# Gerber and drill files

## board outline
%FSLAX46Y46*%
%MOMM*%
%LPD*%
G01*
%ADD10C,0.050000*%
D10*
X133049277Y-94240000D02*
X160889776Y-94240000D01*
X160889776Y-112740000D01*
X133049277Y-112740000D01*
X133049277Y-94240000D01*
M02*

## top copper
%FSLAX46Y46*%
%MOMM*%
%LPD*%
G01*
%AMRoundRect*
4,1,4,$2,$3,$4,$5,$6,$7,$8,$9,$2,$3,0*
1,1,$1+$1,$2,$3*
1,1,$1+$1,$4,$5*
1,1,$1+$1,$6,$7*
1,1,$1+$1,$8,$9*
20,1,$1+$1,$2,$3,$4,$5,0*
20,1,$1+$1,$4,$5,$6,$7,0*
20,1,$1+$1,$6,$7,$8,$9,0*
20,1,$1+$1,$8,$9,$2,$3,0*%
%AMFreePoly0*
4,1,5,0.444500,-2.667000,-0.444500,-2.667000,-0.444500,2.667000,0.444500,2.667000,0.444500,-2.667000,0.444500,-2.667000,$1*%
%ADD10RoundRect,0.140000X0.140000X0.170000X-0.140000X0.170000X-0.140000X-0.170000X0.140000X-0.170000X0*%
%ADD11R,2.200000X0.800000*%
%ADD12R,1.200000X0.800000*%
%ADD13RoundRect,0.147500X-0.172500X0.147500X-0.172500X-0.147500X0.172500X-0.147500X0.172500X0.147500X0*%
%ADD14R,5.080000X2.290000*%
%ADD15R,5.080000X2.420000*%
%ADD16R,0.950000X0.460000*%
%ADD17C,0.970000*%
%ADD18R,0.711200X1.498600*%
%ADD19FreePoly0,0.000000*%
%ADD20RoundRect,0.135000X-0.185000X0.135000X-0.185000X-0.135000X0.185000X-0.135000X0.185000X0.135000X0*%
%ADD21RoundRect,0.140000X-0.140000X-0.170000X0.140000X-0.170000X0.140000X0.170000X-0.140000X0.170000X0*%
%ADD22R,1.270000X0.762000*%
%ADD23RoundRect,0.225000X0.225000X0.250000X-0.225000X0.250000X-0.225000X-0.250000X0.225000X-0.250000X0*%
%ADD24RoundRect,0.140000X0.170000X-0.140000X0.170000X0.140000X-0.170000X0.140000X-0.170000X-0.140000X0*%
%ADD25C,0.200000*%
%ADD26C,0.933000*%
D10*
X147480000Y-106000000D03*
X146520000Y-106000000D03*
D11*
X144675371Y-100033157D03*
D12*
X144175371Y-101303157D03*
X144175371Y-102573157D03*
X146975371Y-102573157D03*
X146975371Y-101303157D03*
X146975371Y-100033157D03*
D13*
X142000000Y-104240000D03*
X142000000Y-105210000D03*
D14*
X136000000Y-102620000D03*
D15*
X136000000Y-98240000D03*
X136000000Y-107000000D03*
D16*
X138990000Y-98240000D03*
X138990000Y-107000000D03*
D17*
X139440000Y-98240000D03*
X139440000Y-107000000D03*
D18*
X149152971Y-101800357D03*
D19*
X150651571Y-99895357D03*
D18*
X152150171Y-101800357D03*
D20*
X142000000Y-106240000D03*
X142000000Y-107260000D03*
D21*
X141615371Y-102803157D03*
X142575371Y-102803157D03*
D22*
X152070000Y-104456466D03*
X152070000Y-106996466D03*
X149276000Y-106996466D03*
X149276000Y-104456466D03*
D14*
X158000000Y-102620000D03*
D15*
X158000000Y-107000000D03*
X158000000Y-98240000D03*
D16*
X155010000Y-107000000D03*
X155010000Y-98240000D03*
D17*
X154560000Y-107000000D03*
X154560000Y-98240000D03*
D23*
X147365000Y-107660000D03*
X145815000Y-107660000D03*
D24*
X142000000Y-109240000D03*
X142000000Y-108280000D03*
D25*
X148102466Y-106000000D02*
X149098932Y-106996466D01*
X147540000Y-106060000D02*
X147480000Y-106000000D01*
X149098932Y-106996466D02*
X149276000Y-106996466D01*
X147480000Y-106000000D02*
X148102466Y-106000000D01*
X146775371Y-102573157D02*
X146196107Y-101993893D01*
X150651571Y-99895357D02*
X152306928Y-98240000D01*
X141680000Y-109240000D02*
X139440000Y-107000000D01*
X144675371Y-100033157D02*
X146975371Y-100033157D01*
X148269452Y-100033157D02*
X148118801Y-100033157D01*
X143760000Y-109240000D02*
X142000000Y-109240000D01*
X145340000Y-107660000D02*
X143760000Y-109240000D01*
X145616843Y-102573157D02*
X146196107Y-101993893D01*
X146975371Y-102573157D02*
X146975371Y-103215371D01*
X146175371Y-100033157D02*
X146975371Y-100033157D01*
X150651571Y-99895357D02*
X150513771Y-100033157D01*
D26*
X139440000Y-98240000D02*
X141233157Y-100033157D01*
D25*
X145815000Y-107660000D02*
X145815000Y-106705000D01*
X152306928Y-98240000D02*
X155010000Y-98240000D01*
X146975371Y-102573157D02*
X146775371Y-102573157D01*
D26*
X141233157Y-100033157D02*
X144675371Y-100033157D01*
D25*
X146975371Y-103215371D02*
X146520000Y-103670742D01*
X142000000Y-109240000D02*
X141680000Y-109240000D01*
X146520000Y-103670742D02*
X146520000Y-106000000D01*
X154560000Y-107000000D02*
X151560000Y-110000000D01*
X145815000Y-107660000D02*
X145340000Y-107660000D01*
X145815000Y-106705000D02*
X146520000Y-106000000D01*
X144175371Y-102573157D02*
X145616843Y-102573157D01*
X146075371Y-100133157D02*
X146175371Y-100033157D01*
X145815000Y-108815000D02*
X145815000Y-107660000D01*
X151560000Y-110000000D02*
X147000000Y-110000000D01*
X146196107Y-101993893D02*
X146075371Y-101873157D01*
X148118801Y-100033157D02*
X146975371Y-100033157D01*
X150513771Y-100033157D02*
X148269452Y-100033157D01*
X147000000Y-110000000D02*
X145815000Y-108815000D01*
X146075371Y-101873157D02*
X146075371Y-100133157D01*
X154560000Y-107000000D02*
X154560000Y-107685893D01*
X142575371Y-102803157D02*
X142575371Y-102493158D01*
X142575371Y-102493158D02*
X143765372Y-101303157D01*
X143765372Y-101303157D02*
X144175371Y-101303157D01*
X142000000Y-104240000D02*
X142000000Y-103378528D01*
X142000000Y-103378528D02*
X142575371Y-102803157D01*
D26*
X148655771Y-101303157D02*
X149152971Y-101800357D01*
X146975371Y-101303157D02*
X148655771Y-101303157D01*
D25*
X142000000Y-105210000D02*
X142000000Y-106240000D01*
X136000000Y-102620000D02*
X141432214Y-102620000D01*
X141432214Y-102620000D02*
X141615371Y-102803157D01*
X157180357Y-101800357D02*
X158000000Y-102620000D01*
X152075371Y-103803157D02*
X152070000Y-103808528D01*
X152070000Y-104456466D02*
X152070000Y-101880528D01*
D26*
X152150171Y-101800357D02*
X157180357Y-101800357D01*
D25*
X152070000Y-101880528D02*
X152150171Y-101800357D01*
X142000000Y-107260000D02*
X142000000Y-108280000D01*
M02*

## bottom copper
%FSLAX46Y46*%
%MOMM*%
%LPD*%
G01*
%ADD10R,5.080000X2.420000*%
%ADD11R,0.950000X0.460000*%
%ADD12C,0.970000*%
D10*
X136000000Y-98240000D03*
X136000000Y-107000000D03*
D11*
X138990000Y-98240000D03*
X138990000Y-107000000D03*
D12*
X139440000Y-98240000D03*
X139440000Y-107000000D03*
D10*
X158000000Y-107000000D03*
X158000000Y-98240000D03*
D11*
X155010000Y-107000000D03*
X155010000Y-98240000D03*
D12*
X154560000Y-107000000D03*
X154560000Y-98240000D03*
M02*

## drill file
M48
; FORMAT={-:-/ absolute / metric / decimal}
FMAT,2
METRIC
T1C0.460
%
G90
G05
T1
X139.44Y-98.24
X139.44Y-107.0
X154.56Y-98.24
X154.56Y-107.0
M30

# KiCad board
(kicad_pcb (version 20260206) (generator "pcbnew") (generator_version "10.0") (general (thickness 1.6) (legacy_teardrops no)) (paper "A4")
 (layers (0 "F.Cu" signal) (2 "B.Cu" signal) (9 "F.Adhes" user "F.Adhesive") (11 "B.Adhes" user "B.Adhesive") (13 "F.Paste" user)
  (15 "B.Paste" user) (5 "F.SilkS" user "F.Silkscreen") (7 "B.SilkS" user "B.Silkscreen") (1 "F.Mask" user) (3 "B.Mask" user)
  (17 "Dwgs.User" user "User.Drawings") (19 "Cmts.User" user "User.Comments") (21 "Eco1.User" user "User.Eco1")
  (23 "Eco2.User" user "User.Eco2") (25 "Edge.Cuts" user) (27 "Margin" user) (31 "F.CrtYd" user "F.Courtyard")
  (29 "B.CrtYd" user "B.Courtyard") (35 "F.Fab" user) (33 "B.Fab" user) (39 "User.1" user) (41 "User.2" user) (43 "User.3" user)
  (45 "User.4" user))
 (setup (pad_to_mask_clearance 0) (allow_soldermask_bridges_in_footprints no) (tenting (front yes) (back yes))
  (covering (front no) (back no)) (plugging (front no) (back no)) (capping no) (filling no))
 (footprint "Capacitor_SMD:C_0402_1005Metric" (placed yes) (layer "F.Cu") (at 147 106 180)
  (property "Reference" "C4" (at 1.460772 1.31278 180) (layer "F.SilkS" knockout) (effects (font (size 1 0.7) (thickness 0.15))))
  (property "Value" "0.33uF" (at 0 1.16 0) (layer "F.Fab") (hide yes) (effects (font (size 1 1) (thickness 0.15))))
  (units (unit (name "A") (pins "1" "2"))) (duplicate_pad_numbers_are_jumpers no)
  (pad "1" smd roundrect (at -0.48 0 180) (size 0.56 0.62) (layers "F.Cu" "F.Mask" "F.Paste") (roundrect_rratio 0.25) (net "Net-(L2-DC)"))
  (pad "2" smd roundrect (at 0.48 0 180) (size 0.56 0.62) (layers "F.Cu" "F.Mask" "F.Paste") (roundrect_rratio 0.25) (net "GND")))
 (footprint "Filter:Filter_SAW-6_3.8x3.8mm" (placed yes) (layer "F.Cu") (at 145.575371 101.303157)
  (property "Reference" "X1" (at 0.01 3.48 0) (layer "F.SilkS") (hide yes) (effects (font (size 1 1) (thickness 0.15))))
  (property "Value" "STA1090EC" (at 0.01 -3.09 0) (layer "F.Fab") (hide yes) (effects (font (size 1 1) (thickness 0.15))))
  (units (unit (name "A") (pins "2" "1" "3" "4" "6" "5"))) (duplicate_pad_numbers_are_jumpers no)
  (pad "1" smd rect (at -0.9 -1.27) (size 2.2 0.8) (layers "F.Cu" "F.Mask" "F.Paste") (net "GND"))
  (pad "2" smd rect (at -1.4 0) (size 1.2 0.8) (layers "F.Cu" "F.Mask" "F.Paste") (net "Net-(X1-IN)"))
  (pad "3" smd rect (at -1.4 1.27) (size 1.2 0.8) (layers "F.Cu" "F.Mask" "F.Paste") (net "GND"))
  (pad "4" smd rect (at 1.4 1.27) (size 1.2 0.8) (layers "F.Cu" "F.Mask" "F.Paste") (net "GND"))
  (pad "5" smd rect (at 1.4 0) (size 1.2 0.8) (layers "F.Cu" "F.Mask" "F.Paste") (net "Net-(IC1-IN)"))
  (pad "6" smd rect (at 1.4 -1.27) (size 1.2 0.8) (layers "F.Cu" "F.Mask" "F.Paste") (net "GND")))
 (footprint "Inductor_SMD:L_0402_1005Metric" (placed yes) (layer "F.Cu") (at 142 104.725 -90)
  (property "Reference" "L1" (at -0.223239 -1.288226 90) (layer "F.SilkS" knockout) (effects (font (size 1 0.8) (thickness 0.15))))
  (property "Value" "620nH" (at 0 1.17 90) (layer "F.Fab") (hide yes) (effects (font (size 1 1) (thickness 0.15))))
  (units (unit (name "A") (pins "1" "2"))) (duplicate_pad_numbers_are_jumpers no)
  (pad "1" smd roundrect (at -0.485 0 270) (size 0.59 0.64) (layers "F.Cu" "F.Mask" "F.Paste") (roundrect_rratio 0.25) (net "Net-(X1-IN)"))
  (pad "2" smd roundrect (at 0.485 0 270) (size 0.59 0.64) (layers "F.Cu" "F.Mask" "F.Paste") (roundrect_rratio 0.25) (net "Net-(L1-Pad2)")))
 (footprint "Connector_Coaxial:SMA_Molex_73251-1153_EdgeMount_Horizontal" (layer "F.Cu") (at 137.72 102.62)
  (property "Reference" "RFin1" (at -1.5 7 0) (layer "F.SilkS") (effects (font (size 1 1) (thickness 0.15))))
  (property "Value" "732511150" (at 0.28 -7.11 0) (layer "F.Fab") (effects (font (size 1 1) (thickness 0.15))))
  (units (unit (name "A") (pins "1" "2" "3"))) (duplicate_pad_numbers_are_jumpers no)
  (pad "1" smd rect (at -1.72 0) (size 5.08 2.29) (layers "F.Cu" "F.Mask" "F.Paste") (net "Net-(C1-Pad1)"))
  (pad "2" smd rect (at -1.72 -4.38) (size 5.08 2.42) (layers "F.Cu" "F.Mask" "F.Paste") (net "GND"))
  (pad "2" smd rect (at -1.72 -4.38) (size 5.08 2.42) (layers "B.Cu" "B.Mask" "B.Paste") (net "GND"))
  (pad "2" smd rect (at -1.72 4.38) (size 5.08 2.42) (layers "F.Cu" "F.Mask" "F.Paste") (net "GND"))
  (pad "2" smd rect (at -1.72 4.38) (size 5.08 2.42) (layers "B.Cu" "B.Mask" "B.Paste") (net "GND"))
  (pad "2" smd rect (at 1.27 -4.38) (size 0.95 0.46) (layers "F.Cu") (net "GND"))
  (pad "2" smd rect (at 1.27 -4.38) (size 0.95 0.46) (layers "B.Cu") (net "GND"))
  (pad "2" smd rect (at 1.27 4.38) (size 0.95 0.46) (layers "F.Cu") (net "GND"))
  (pad "2" smd rect (at 1.27 4.38) (size 0.95 0.46) (layers "B.Cu") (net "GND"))
  (pad "2" thru_hole circle (at 1.72 -4.38) (size 0.97 0.97) (drill 0.46) (layers "*.Cu") (remove_unused_layers no) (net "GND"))
  (pad "2" thru_hole circle (at 1.72 4.38) (size 0.97 0.97) (drill 0.46) (layers "*.Cu") (remove_unused_layers no) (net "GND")))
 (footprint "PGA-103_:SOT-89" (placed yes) (layer "F.Cu") (at 150.575371 98.803157)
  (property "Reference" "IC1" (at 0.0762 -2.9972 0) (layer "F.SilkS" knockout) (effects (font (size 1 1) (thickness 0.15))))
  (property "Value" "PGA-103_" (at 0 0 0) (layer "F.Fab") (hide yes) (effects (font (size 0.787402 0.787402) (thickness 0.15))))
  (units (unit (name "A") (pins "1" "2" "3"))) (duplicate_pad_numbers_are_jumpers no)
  (pad "1" smd rect (at -1.4224 2.9972) (size 0.7112 1.4986) (layers "F.Cu" "F.Mask" "F.Paste") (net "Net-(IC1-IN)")
   (solder_mask_margin 0.102))
  (pad "2" smd custom (at 0.0762 1.0922) (size 0.889 5.334) (layers "F.Cu" "F.Mask" "F.Paste") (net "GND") (solder_mask_margin 0.102)
   (options (clearance outline) (anchor rect)) (primitives))
  (pad "3" smd rect (at 1.5748 2.9972) (size 0.7112 1.4986) (layers "F.Cu" "F.Mask" "F.Paste") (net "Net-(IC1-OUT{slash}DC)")
   (solder_mask_margin 0.102)))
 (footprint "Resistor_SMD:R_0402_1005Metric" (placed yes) (layer "F.Cu") (at 142 106.75 -90)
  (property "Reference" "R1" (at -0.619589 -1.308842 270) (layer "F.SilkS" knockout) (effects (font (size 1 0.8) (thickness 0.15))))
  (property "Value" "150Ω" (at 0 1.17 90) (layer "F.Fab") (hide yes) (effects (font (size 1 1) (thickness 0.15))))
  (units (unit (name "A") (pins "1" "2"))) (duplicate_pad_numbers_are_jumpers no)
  (pad "1" smd roundrect (at -0.51 0 270) (size 0.54 0.64) (layers "F.Cu" "F.Mask" "F.Paste") (roundrect_rratio 0.25) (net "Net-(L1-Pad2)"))
  (pad "2" smd roundrect (at 0.51 0 270) (size 0.54 0.64) (layers "F.Cu" "F.Mask" "F.Paste") (roundrect_rratio 0.25) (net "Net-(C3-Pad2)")))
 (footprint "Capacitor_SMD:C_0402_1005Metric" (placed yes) (layer "F.Cu") (at 142.095371 102.803157)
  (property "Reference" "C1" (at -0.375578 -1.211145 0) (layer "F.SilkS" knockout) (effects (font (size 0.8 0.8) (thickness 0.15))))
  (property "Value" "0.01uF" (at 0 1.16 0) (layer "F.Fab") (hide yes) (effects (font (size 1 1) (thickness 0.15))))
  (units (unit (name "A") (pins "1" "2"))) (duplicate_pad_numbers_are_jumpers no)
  (pad "1" smd roundrect (at -0.48 0) (size 0.56 0.62) (layers "F.Cu" "F.Mask" "F.Paste") (roundrect_rratio 0.25) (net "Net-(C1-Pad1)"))
  (pad "2" smd roundrect (at 0.48 0) (size 0.56 0.62) (layers "F.Cu" "F.Mask" "F.Paste") (roundrect_rratio 0.25) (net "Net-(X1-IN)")))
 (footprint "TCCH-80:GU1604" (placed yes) (layer "F.Cu") (at 150.673 105.726466 -90)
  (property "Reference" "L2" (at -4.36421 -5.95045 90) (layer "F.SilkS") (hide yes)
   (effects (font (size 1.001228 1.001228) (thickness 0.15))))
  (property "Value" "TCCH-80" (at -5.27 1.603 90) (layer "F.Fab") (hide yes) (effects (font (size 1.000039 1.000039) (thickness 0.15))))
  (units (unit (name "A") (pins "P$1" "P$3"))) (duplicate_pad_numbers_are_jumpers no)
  (pad "P$1" smd rect (at -1.27 -1.397 270) (size 0.762 1.27) (layers "F.Cu" "F.Mask" "F.Paste") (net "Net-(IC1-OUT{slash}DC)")
   (solder_mask_margin 0.102))
  (pad "P$2" smd rect (at 1.27 -1.397 270) (size 0.762 1.27) (layers "F.Cu" "F.Mask" "F.Paste") (solder_mask_margin 0.102))
  (pad "P$3" smd rect (at 1.27 1.397 270) (size 0.762 1.27) (layers "F.Cu" "F.Mask" "F.Paste") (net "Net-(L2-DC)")
   (solder_mask_margin 0.102))
  (pad "P$4" smd rect (at -1.27 1.397 270) (size 0.762 1.27) (layers "F.Cu" "F.Mask" "F.Paste") (solder_mask_margin 0.102)))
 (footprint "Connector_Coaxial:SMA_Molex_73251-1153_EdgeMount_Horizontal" (layer "F.Cu") (at 156.28 102.62 180)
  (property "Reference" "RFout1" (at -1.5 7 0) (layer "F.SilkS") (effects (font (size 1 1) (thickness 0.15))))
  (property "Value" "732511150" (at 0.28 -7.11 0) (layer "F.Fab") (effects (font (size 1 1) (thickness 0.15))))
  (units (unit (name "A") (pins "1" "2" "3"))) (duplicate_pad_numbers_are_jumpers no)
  (pad "1" smd rect (at -1.72 0 180) (size 5.08 2.29) (layers "F.Cu" "F.Mask" "F.Paste") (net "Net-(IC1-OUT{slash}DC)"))
  (pad "2" smd rect (at -1.72 -4.38 180) (size 5.08 2.42) (layers "F.Cu" "F.Mask" "F.Paste") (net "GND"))
  (pad "2" smd rect (at -1.72 -4.38 180) (size 5.08 2.42) (layers "B.Cu" "B.Mask" "B.Paste") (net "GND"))
  (pad "2" smd rect (at -1.72 4.38 180) (size 5.08 2.42) (layers "F.Cu" "F.Mask" "F.Paste") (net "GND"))
  (pad "2" smd rect (at -1.72 4.38 180) (size 5.08 2.42) (layers "B.Cu" "B.Mask" "B.Paste") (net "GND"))
  (pad "2" smd rect (at 1.27 -4.38 180) (size 0.95 0.46) (layers "F.Cu") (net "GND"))
  (pad "2" smd rect (at 1.27 -4.38 180) (size 0.95 0.46) (layers "B.Cu") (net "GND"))
  (pad "2" smd rect (at 1.27 4.38 180) (size 0.95 0.46) (layers "F.Cu") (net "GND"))
  (pad "2" smd rect (at 1.27 4.38 180) (size 0.95 0.46) (layers "B.Cu") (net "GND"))
  (pad "2" thru_hole circle (at 1.72 -4.38 180) (size 0.97 0.97) (drill 0.46) (layers "*.Cu") (remove_unused_layers no) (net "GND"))
  (pad "2" thru_hole circle (at 1.72 4.38 180) (size 0.97 0.97) (drill 0.46) (layers "*.Cu") (remove_unused_layers no) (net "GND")))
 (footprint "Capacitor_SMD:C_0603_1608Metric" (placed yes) (layer "F.Cu") (at 146.59 107.66 180)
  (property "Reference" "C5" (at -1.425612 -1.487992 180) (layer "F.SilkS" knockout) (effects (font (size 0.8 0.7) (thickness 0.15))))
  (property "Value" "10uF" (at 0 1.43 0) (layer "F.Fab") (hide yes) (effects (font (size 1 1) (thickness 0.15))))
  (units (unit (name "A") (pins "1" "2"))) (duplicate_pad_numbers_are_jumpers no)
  (pad "1" smd roundrect (at -0.775 0 180) (size 0.9 0.95) (layers "F.Cu" "F.Mask" "F.Paste") (roundrect_rratio 0.25) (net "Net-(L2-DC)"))
  (pad "2" smd roundrect (at 0.775 0 180) (size 0.9 0.95) (layers "F.Cu" "F.Mask" "F.Paste") (roundrect_rratio 0.25) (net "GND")))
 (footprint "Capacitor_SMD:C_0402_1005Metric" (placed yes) (layer "F.Cu") (at 142 108.76 90)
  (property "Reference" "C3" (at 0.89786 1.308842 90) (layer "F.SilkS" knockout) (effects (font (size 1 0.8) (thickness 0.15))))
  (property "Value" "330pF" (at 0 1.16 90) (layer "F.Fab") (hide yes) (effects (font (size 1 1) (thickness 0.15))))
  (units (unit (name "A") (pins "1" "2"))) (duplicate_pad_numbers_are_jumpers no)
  (pad "1" smd roundrect (at -0.48 0 90) (size 0.56 0.62) (layers "F.Cu" "F.Mask" "F.Paste") (roundrect_rratio 0.25) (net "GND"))
  (pad "2" smd roundrect (at 0.48 0 90) (size 0.56 0.62) (layers "F.Cu" "F.Mask" "F.Paste") (roundrect_rratio 0.25) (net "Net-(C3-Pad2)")))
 (gr_rect (start 133.049277 94.24) (end 160.889776 112.74) (stroke (width 0.05) (type default)) (fill no) (layer "Edge.Cuts"))
 (segment (start 148.102466 106) (end 149.098932 106.996466) (width 0.2) (layer "F.Cu") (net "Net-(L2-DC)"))
 (segment (start 147.54 106.06) (end 147.48 106) (width 0.2) (layer "F.Cu") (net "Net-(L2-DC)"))
 (segment (start 149.098932 106.996466) (end 149.276 106.996466) (width 0.2) (layer "F.Cu") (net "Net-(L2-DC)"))
 (segment (start 147.48 106) (end 148.102466 106) (width 0.2) (layer "F.Cu") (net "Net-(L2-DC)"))
 (segment (start 146.775371 102.573157) (end 146.196107 101.993893) (width 0.2) (layer "F.Cu") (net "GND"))
 (segment (start 150.651571 99.895357) (end 152.306928 98.24) (width 0.2) (layer "F.Cu") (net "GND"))
 (segment (start 141.68 109.24) (end 139.44 107) (width 0.2) (layer "F.Cu") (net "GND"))
 (segment (start 144.675371 100.033157) (end 146.975371 100.033157) (width 0.2) (layer "F.Cu") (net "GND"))
 (segment (start 148.269452 100.033157) (end 148.118801 100.033157) (width 0.2) (layer "F.Cu") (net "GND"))
 (segment (start 143.76 109.24) (end 142 109.24) (width 0.2) (layer "F.Cu") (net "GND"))
 (segment (start 145.34 107.66) (end 143.76 109.24) (width 0.2) (layer "F.Cu") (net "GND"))
 (segment (start 145.616843 102.573157) (end 146.196107 101.993893) (width 0.2) (layer "F.Cu") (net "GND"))
 (segment (start 146.975371 102.573157) (end 146.975371 103.215371) (width 0.2) (layer "F.Cu") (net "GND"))
 (segment (start 146.175371 100.033157) (end 146.975371 100.033157) (width 0.2) (layer "F.Cu") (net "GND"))
 (segment (start 150.651571 99.895357) (end 150.513771 100.033157) (width 0.2) (layer "F.Cu") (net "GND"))
 (segment (start 139.44 98.24) (end 141.233157 100.033157) (width 0.933) (layer "F.Cu") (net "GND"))
 (segment (start 145.815 107.66) (end 145.815 106.705) (width 0.2) (layer "F.Cu") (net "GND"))
 (segment (start 152.306928 98.24) (end 155.01 98.24) (width 0.2) (layer "F.Cu") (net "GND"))
 (segment (start 146.975371 102.573157) (end 146.775371 102.573157) (width 0.2) (layer "F.Cu") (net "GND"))
 (segment (start 141.233157 100.033157) (end 144.675371 100.033157) (width 0.933) (layer "F.Cu") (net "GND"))
 (segment (start 146.975371 103.215371) (end 146.52 103.670742) (width 0.2) (layer "F.Cu") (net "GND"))
 (segment (start 142 109.24) (end 141.68 109.24) (width 0.2) (layer "F.Cu") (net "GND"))
 (segment (start 146.52 103.670742) (end 146.52 106) (width 0.2) (layer "F.Cu") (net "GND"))
 (segment (start 154.56 107) (end 151.56 110) (width 0.2) (layer "F.Cu") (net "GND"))
 (segment (start 145.815 107.66) (end 145.34 107.66) (width 0.2) (layer "F.Cu") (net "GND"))
 (segment (start 145.815 106.705) (end 146.52 106) (width 0.2) (layer "F.Cu") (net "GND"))
 (segment (start 144.175371 102.573157) (end 145.616843 102.573157) (width 0.2) (layer "F.Cu") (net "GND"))
 (segment (start 146.075371 100.133157) (end 146.175371 100.033157) (width 0.2) (layer "F.Cu") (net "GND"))
 (segment (start 145.815 108.815) (end 145.815 107.66) (width 0.2) (layer "F.Cu") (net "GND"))
 (segment (start 151.56 110) (end 147 110) (width 0.2) (layer "F.Cu") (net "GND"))
 (segment (start 146.196107 101.993893) (end 146.075371 101.873157) (width 0.2) (layer "F.Cu") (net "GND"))
 (segment (start 148.118801 100.033157) (end 146.975371 100.033157) (width 0.2) (layer "F.Cu") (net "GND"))
 (segment (start 150.513771 100.033157) (end 148.269452 100.033157) (width 0.2) (layer "F.Cu") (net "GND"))
 (segment (start 147 110) (end 145.815 108.815) (width 0.2) (layer "F.Cu") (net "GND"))
 (segment (start 146.075371 101.873157) (end 146.075371 100.133157) (width 0.2) (layer "F.Cu") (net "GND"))
 (segment (start 154.56 107) (end 154.56 107.685893) (width 0.2) (layer "F.Cu") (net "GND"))
 (segment (start 142.575371 102.803157) (end 142.575371 102.493158) (width 0.2) (layer "F.Cu") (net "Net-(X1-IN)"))
 (segment (start 142.575371 102.493158) (end 143.765372 101.303157) (width 0.2) (layer "F.Cu") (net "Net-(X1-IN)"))
 (segment (start 143.765372 101.303157) (end 144.175371 101.303157) (width 0.2) (layer "F.Cu") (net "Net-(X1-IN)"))
 (segment (start 142 104.24) (end 142 103.378528) (width 0.2) (layer "F.Cu") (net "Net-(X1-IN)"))
 (segment (start 142 103.378528) (end 142.575371 102.803157) (width 0.2) (layer "F.Cu") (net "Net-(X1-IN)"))
 (segment (start 148.655771 101.303157) (end 149.152971 101.800357) (width 0.933) (layer "F.Cu") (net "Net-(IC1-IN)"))
 (segment (start 146.975371 101.303157) (end 148.655771 101.303157) (width 0.933) (layer "F.Cu") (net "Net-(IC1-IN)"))
 (segment (start 142 105.21) (end 142 106.24) (width 0.2) (layer "F.Cu") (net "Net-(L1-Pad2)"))
 (segment (start 136 102.62) (end 141.432214 102.62) (width 0.2) (layer "F.Cu") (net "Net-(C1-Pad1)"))
 (segment (start 141.432214 102.62) (end 141.615371 102.803157) (width 0.2) (layer "F.Cu") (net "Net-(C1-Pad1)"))
 (segment (start 157.180357 101.800357) (end 158 102.62) (width 0.2) (layer "F.Cu") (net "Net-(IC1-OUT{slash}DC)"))
 (segment (start 152.075371 103.803157) (end 152.07 103.808528) (width 0.2) (layer "F.Cu") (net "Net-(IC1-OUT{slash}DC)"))
 (segment (start 152.07 104.456466) (end 152.07 101.880528) (width 0.2) (layer "F.Cu") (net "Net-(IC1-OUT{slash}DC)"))
 (segment (start 152.150171 101.800357) (end 157.180357 101.800357) (width 0.933) (layer "F.Cu") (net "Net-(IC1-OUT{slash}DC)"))
 (segment (start 152.07 101.880528) (end 152.150171 101.800357) (width 0.2) (layer "F.Cu") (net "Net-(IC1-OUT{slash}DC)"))
 (segment (start 142 107.26) (end 142 108.28) (width 0.2) (layer "F.Cu") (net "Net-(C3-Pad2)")))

